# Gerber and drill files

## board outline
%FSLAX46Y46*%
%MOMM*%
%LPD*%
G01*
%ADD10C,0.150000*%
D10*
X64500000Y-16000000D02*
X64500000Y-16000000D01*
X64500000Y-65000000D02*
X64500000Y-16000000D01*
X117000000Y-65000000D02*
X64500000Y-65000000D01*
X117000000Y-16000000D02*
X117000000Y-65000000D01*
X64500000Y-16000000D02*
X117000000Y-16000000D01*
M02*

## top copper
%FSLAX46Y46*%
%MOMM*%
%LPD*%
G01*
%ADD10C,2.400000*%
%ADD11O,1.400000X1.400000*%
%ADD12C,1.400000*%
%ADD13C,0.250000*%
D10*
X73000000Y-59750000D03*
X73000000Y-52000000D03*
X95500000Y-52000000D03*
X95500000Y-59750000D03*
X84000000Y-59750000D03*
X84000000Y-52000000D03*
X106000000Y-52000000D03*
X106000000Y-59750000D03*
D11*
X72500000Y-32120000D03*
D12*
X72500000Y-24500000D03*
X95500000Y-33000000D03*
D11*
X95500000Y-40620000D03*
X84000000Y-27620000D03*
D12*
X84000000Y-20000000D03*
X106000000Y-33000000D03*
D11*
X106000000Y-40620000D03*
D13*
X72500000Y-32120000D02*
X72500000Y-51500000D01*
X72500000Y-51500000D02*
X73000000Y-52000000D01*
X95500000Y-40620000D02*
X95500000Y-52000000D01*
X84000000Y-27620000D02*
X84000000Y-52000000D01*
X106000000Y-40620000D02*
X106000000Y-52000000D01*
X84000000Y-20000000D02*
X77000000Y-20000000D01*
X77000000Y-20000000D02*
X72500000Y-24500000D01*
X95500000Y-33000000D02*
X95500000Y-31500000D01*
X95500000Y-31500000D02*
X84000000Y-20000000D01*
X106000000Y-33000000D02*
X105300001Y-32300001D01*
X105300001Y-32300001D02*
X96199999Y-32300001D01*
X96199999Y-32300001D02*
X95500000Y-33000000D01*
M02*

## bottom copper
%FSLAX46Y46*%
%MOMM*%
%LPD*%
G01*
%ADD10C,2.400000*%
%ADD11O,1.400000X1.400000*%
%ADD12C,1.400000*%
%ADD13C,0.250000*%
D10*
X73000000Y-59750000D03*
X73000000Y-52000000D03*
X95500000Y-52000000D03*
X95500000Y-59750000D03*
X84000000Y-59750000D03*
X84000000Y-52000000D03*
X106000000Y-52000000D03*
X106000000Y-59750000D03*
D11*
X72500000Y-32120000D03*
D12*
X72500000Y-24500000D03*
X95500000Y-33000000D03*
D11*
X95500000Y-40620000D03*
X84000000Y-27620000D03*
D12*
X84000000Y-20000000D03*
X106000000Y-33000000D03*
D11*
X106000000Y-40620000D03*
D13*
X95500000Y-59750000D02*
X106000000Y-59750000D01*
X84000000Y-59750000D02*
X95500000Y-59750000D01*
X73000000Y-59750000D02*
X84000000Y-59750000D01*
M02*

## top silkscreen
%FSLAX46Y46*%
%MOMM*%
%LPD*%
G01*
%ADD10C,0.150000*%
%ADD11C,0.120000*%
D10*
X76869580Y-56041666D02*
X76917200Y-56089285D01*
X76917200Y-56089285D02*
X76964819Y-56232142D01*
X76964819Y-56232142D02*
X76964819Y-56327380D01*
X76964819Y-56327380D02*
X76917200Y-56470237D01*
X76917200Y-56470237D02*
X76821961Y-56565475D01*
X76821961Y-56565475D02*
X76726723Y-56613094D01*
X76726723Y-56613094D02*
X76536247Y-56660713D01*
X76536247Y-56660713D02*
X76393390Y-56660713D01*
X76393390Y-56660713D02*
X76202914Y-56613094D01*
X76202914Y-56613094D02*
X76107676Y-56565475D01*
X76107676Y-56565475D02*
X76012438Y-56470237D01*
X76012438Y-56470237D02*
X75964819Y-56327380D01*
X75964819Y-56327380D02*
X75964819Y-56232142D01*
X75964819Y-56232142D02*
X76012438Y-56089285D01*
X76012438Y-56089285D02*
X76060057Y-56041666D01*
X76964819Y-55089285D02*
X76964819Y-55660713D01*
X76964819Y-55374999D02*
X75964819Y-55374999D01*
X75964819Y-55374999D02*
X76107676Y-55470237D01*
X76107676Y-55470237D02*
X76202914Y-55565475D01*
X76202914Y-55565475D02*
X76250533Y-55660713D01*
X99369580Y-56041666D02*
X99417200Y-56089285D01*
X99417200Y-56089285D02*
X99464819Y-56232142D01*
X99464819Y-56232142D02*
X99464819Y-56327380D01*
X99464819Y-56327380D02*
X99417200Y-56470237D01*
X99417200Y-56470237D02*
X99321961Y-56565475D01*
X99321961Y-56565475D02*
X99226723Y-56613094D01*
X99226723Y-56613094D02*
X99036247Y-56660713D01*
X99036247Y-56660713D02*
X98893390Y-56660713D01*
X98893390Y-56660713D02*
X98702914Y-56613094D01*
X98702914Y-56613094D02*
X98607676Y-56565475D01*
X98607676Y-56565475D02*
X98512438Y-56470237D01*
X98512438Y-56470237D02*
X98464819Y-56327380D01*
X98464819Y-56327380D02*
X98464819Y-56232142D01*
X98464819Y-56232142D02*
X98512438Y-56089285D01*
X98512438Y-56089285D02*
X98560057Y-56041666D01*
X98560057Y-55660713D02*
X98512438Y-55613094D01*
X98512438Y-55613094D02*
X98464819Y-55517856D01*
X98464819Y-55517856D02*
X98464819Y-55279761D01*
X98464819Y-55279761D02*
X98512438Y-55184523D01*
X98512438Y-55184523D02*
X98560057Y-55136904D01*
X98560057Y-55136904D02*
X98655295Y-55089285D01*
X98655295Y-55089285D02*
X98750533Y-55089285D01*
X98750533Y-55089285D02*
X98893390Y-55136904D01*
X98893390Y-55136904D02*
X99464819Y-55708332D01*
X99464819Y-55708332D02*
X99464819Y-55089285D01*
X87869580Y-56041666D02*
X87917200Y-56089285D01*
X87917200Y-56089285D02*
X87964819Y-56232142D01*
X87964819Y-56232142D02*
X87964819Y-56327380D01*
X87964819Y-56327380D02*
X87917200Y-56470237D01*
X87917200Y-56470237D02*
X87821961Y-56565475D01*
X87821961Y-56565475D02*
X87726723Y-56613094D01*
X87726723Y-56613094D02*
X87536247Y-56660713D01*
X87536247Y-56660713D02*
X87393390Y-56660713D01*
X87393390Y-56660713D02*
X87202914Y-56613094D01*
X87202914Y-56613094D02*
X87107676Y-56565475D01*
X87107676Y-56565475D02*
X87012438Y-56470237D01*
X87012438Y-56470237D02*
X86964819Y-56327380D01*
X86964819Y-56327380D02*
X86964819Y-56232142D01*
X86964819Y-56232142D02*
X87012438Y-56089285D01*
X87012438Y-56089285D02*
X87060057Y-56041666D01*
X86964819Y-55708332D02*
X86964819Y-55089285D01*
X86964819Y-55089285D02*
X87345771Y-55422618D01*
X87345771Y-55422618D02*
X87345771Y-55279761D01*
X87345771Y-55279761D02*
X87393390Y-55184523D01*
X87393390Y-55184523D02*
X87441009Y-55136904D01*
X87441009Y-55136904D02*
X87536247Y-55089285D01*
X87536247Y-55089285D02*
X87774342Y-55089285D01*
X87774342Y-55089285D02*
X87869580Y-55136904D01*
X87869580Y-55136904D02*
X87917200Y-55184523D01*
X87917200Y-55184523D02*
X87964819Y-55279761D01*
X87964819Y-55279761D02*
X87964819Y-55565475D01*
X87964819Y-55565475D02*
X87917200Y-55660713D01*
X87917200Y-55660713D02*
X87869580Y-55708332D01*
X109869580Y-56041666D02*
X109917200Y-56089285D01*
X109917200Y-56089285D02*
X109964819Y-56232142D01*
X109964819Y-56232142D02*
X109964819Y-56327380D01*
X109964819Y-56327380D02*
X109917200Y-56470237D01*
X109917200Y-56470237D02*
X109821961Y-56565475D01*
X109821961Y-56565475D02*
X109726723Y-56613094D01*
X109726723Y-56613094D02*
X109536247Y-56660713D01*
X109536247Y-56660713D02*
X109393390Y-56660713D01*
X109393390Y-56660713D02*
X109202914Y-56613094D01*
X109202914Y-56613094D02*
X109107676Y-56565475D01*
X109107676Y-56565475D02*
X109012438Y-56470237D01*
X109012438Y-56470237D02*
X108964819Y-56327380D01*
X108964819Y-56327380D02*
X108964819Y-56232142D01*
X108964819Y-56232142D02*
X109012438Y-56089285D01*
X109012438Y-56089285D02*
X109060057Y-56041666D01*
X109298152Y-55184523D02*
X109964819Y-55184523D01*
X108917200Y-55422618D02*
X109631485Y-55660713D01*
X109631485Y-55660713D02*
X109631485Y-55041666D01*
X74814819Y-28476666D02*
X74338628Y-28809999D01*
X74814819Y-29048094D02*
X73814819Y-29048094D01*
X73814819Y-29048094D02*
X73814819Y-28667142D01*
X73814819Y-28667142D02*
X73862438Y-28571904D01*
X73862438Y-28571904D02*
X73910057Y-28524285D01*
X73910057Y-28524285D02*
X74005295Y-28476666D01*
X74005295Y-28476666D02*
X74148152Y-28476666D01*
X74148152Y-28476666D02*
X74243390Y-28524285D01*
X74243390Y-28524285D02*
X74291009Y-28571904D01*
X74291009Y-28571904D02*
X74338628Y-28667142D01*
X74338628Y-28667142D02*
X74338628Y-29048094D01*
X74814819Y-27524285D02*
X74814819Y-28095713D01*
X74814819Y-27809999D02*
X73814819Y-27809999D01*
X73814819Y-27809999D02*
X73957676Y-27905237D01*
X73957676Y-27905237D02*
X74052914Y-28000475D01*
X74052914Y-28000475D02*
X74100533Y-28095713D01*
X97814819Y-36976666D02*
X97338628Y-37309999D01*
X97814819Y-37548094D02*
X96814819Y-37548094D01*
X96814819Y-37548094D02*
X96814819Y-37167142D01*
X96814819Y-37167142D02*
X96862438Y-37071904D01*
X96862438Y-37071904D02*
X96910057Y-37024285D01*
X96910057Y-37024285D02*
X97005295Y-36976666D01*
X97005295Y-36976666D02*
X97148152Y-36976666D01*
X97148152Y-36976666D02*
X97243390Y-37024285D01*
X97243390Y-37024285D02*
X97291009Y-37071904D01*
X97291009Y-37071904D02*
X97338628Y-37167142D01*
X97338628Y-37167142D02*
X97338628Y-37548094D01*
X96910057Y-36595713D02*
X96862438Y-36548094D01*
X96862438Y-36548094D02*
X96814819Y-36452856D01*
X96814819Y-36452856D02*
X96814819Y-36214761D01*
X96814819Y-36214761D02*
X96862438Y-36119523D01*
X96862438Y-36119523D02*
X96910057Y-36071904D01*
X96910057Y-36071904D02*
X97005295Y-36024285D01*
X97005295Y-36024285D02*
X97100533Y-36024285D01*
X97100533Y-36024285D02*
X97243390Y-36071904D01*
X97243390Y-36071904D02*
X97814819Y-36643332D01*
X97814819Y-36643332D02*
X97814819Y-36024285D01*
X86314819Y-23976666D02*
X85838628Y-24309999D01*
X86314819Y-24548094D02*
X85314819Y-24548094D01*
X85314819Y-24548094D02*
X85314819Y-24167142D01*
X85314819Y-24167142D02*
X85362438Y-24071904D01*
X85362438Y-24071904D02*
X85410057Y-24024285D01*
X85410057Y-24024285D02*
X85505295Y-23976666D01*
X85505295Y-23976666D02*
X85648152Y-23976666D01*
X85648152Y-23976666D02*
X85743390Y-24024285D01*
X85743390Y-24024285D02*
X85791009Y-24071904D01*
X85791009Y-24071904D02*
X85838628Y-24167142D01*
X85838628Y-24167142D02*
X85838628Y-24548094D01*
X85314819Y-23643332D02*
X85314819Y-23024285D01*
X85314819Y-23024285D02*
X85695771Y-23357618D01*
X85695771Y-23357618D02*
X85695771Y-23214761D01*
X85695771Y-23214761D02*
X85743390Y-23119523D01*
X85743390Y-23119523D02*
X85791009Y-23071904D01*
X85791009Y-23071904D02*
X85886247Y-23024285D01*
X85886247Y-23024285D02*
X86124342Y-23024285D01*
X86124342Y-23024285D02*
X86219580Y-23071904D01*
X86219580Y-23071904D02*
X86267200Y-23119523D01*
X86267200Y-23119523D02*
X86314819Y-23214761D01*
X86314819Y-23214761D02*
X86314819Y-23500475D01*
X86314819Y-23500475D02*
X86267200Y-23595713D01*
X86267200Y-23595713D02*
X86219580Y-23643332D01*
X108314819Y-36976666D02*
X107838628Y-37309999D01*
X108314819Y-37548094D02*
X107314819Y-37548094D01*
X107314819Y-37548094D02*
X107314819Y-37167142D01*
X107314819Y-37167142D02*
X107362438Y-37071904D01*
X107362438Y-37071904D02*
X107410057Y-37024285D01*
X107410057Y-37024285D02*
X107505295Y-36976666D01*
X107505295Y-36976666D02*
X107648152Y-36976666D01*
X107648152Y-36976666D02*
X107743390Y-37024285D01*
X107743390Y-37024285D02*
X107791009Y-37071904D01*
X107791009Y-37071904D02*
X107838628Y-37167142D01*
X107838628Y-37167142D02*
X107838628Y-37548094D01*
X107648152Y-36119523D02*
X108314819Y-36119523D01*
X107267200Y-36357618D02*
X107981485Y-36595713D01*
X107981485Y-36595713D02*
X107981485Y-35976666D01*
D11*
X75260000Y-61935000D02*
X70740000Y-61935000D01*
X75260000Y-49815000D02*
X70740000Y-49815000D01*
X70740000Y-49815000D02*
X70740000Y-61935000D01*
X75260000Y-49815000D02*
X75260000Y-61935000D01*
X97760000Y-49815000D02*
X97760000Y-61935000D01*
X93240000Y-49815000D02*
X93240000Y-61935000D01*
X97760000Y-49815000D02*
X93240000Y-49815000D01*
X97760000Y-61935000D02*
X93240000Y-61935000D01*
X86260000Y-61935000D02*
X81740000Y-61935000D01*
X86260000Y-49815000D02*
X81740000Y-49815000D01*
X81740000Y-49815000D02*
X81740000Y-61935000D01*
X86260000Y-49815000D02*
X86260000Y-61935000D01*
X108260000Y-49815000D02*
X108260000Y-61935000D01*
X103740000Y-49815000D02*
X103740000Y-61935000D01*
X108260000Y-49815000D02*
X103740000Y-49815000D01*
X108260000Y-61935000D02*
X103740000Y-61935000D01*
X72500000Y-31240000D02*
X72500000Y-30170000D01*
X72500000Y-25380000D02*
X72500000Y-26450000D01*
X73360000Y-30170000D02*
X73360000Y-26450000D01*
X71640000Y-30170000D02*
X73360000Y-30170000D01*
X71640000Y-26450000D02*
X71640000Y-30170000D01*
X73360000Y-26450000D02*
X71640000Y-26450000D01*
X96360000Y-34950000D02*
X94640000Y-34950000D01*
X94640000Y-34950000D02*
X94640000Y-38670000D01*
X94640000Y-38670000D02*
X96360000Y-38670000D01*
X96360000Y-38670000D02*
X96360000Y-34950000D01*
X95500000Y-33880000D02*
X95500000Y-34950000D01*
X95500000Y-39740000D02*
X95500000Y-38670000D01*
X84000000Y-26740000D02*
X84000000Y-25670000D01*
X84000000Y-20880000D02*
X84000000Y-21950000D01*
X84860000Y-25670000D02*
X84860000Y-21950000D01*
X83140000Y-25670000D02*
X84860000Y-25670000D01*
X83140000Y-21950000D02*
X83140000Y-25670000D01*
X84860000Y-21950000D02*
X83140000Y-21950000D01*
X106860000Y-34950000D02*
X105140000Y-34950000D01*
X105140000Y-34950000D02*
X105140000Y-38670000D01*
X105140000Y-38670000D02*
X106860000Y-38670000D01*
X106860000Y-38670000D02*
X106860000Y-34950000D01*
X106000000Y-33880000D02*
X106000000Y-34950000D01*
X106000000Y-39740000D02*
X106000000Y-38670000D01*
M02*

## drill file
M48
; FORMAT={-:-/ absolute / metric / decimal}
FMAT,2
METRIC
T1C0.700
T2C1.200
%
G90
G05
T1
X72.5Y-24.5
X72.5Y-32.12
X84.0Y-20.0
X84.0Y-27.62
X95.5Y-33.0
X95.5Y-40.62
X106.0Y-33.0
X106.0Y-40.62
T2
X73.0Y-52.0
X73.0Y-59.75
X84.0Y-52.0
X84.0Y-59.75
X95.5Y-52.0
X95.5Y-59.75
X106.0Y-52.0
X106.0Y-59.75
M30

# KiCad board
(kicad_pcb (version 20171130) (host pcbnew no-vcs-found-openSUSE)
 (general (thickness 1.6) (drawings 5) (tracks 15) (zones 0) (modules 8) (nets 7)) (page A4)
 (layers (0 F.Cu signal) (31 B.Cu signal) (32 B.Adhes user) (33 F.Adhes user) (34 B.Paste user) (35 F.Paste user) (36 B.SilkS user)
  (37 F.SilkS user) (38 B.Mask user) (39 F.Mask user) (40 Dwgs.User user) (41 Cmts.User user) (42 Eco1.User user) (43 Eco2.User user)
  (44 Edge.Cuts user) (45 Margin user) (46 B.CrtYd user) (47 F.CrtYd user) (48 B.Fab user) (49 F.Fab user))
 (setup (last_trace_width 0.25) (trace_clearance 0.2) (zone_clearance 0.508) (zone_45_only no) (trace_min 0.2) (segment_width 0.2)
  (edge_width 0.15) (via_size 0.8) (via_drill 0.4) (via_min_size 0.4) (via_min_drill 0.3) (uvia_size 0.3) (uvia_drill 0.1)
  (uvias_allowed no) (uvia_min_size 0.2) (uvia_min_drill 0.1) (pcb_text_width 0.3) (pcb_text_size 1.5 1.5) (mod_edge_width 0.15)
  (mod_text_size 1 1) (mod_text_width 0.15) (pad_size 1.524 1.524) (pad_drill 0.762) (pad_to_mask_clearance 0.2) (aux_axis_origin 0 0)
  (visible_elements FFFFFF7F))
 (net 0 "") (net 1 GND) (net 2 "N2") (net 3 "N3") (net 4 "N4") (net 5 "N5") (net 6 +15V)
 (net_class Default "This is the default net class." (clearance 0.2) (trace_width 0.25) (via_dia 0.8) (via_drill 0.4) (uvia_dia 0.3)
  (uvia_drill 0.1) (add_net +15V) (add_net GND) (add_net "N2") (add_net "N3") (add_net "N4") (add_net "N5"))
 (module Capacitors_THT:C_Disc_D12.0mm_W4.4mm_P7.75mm (layer F.Cu) (at 73 52 270)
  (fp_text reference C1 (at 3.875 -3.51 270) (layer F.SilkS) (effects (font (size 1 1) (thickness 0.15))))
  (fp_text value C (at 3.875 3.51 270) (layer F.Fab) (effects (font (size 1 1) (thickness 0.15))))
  (fp_line (start 9.935 -2.26) (end 9.935 2.26) (layer F.SilkS) (width 0.12))
  (fp_line (start -2.185 -2.26) (end -2.185 2.26) (layer F.SilkS) (width 0.12))
  (fp_line (start -2.185 2.26) (end 9.935 2.26) (layer F.SilkS) (width 0.12))
  (fp_line (start -2.185 -2.26) (end 9.935 -2.26) (layer F.SilkS) (width 0.12))
  (pad 2 thru_hole circle (at 7.75 0 270) (size 2.4 2.4) (drill 1.2) (layers *.Cu *.Mask) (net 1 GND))
  (pad 1 thru_hole circle (at 0 0 270) (size 2.4 2.4) (drill 1.2) (layers *.Cu *.Mask) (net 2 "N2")))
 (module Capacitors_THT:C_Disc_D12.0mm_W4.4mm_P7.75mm (layer F.Cu) (at 95.5 52 270)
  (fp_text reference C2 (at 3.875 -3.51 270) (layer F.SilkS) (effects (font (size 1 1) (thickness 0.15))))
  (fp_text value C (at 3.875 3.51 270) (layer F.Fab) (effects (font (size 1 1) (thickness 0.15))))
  (fp_line (start -2.185 -2.26) (end 9.935 -2.26) (layer F.SilkS) (width 0.12))
  (fp_line (start -2.185 2.26) (end 9.935 2.26) (layer F.SilkS) (width 0.12))
  (fp_line (start -2.185 -2.26) (end -2.185 2.26) (layer F.SilkS) (width 0.12))
  (fp_line (start 9.935 -2.26) (end 9.935 2.26) (layer F.SilkS) (width 0.12))
  (pad 1 thru_hole circle (at 0 0 270) (size 2.4 2.4) (drill 1.2) (layers *.Cu *.Mask) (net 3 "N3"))
  (pad 2 thru_hole circle (at 7.75 0 270) (size 2.4 2.4) (drill 1.2) (layers *.Cu *.Mask) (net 1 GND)))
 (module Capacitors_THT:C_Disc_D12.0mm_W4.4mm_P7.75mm (layer F.Cu) (at 84 52 270)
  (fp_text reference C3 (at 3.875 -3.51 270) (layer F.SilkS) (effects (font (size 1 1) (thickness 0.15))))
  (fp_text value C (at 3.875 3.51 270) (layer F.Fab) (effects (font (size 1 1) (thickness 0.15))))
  (fp_line (start 9.935 -2.26) (end 9.935 2.26) (layer F.SilkS) (width 0.12))
  (fp_line (start -2.185 -2.26) (end -2.185 2.26) (layer F.SilkS) (width 0.12))
  (fp_line (start -2.185 2.26) (end 9.935 2.26) (layer F.SilkS) (width 0.12))
  (fp_line (start -2.185 -2.26) (end 9.935 -2.26) (layer F.SilkS) (width 0.12))
  (pad 2 thru_hole circle (at 7.75 0 270) (size 2.4 2.4) (drill 1.2) (layers *.Cu *.Mask) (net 1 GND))
  (pad 1 thru_hole circle (at 0 0 270) (size 2.4 2.4) (drill 1.2) (layers *.Cu *.Mask) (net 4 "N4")))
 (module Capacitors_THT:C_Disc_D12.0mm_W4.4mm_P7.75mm (layer F.Cu) (at 106 52 270)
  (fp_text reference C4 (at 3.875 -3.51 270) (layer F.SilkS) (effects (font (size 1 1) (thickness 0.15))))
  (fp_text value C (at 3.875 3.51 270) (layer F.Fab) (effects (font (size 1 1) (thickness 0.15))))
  (fp_line (start -2.185 -2.26) (end 9.935 -2.26) (layer F.SilkS) (width 0.12))
  (fp_line (start -2.185 2.26) (end 9.935 2.26) (layer F.SilkS) (width 0.12))
  (fp_line (start -2.185 -2.26) (end -2.185 2.26) (layer F.SilkS) (width 0.12))
  (fp_line (start 9.935 -2.26) (end 9.935 2.26) (layer F.SilkS) (width 0.12))
  (pad 1 thru_hole circle (at 0 0 270) (size 2.4 2.4) (drill 1.2) (layers *.Cu *.Mask) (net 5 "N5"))
  (pad 2 thru_hole circle (at 7.75 0 270) (size 2.4 2.4) (drill 1.2) (layers *.Cu *.Mask) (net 1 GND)))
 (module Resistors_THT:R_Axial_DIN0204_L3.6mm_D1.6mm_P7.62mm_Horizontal (layer F.Cu) (at 72.5 24.5 270)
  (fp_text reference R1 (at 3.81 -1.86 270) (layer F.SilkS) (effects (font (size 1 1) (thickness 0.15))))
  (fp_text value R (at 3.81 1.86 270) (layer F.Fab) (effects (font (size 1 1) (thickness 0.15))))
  (fp_line (start 6.74 0) (end 5.67 0) (layer F.SilkS) (width 0.12))
  (fp_line (start 0.88 0) (end 1.95 0) (layer F.SilkS) (width 0.12))
  (fp_line (start 5.67 -0.86) (end 1.95 -0.86) (layer F.SilkS) (width 0.12))
  (fp_line (start 5.67 0.86) (end 5.67 -0.86) (layer F.SilkS) (width 0.12))
  (fp_line (start 1.95 0.86) (end 5.67 0.86) (layer F.SilkS) (width 0.12))
  (fp_line (start 1.95 -0.86) (end 1.95 0.86) (layer F.SilkS) (width 0.12))
  (pad 2 thru_hole oval (at 7.62 0 270) (size 1.4 1.4) (drill 0.7) (layers *.Cu *.Mask) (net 2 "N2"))
  (pad 1 thru_hole circle (at 0 0 270) (size 1.4 1.4) (drill 0.7) (layers *.Cu *.Mask) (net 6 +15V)))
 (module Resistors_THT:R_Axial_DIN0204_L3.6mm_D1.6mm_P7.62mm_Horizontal (layer F.Cu) (at 95.5 33 270)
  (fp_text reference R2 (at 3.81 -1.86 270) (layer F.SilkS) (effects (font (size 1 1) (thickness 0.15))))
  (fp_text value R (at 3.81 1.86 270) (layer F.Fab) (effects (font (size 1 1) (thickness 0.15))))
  (fp_line (start 1.95 -0.86) (end 1.95 0.86) (layer F.SilkS) (width 0.12))
  (fp_line (start 1.95 0.86) (end 5.67 0.86) (layer F.SilkS) (width 0.12))
  (fp_line (start 5.67 0.86) (end 5.67 -0.86) (layer F.SilkS) (width 0.12))
  (fp_line (start 5.67 -0.86) (end 1.95 -0.86) (layer F.SilkS) (width 0.12))
  (fp_line (start 0.88 0) (end 1.95 0) (layer F.SilkS) (width 0.12))
  (fp_line (start 6.74 0) (end 5.67 0) (layer F.SilkS) (width 0.12))
  (pad 1 thru_hole circle (at 0 0 270) (size 1.4 1.4) (drill 0.7) (layers *.Cu *.Mask) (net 6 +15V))
  (pad 2 thru_hole oval (at 7.62 0 270) (size 1.4 1.4) (drill 0.7) (layers *.Cu *.Mask) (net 3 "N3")))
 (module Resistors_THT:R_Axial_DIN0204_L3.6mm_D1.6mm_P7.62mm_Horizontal (layer F.Cu) (at 84 20 270)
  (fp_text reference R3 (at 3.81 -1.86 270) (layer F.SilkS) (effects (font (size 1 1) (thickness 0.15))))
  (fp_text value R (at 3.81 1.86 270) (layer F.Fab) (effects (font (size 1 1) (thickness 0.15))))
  (fp_line (start 6.74 0) (end 5.67 0) (layer F.SilkS) (width 0.12))
  (fp_line (start 0.88 0) (end 1.95 0) (layer F.SilkS) (width 0.12))
  (fp_line (start 5.67 -0.86) (end 1.95 -0.86) (layer F.SilkS) (width 0.12))
  (fp_line (start 5.67 0.86) (end 5.67 -0.86) (layer F.SilkS) (width 0.12))
  (fp_line (start 1.95 0.86) (end 5.67 0.86) (layer F.SilkS) (width 0.12))
  (fp_line (start 1.95 -0.86) (end 1.95 0.86) (layer F.SilkS) (width 0.12))
  (pad 2 thru_hole oval (at 7.62 0 270) (size 1.4 1.4) (drill 0.7) (layers *.Cu *.Mask) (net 4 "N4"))
  (pad 1 thru_hole circle (at 0 0 270) (size 1.4 1.4) (drill 0.7) (layers *.Cu *.Mask) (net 6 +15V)))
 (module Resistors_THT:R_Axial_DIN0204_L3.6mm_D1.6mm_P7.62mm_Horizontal (layer F.Cu) (at 106 33 270)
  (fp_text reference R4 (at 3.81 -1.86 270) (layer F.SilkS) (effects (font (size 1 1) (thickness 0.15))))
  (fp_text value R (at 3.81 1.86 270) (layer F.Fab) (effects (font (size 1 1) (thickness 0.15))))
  (fp_line (start 1.95 -0.86) (end 1.95 0.86) (layer F.SilkS) (width 0.12))
  (fp_line (start 1.95 0.86) (end 5.67 0.86) (layer F.SilkS) (width 0.12))
  (fp_line (start 5.67 0.86) (end 5.67 -0.86) (layer F.SilkS) (width 0.12))
  (fp_line (start 5.67 -0.86) (end 1.95 -0.86) (layer F.SilkS) (width 0.12))
  (fp_line (start 0.88 0) (end 1.95 0) (layer F.SilkS) (width 0.12))
  (fp_line (start 6.74 0) (end 5.67 0) (layer F.SilkS) (width 0.12))
  (pad 1 thru_hole circle (at 0 0 270) (size 1.4 1.4) (drill 0.7) (layers *.Cu *.Mask) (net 6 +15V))
  (pad 2 thru_hole oval (at 7.62 0 270) (size 1.4 1.4) (drill 0.7) (layers *.Cu *.Mask) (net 5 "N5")))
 (gr_line (start 64.5 16) (end 64.5 16) (layer Edge.Cuts) (width 0.15))
 (gr_line (start 64.5 65) (end 64.5 16) (layer Edge.Cuts) (width 0.15))
 (gr_line (start 117 65) (end 64.5 65) (layer Edge.Cuts) (width 0.15))
 (gr_line (start 117 16) (end 117 65) (layer Edge.Cuts) (width 0.15))
 (gr_line (start 64.5 16) (end 117 16) (layer Edge.Cuts) (width 0.15))
 (segment (start 95.5 59.75) (end 106 59.75) (width 0.25) (layer B.Cu) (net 1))
 (segment (start 84 59.75) (end 95.5 59.75) (width 0.25) (layer B.Cu) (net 1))
 (segment (start 73 59.75) (end 84 59.75) (width 0.25) (layer B.Cu) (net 1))
 (segment (start 72.5 32.12) (end 72.5 51.5) (width 0.25) (layer F.Cu) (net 2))
 (segment (start 72.5 51.5) (end 73 52) (width 0.25) (layer F.Cu) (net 2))
 (segment (start 95.5 40.62) (end 95.5 52) (width 0.25) (layer F.Cu) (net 3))
 (segment (start 84 27.62) (end 84 52) (width 0.25) (layer F.Cu) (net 4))
 (segment (start 106 40.62) (end 106 52) (width 0.25) (layer F.Cu) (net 5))
 (segment (start 84 20) (end 77 20) (width 0.25) (layer F.Cu) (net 6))
 (segment (start 77 20) (end 72.5 24.5) (width 0.25) (layer F.Cu) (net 6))
 (segment (start 95.5 33) (end 95.5 31.5) (width 0.25) (layer F.Cu) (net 6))
 (segment (start 95.5 31.5) (end 84 20) (width 0.25) (layer F.Cu) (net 6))
 (segment (start 106 33) (end 105.300001 32.300001) (width 0.25) (layer F.Cu) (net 6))
 (segment (start 105.300001 32.300001) (end 96.199999 32.300001) (width 0.25) (layer F.Cu) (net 6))
 (segment (start 96.199999 32.300001) (end 95.5 33) (width 0.25) (layer F.Cu) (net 6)))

